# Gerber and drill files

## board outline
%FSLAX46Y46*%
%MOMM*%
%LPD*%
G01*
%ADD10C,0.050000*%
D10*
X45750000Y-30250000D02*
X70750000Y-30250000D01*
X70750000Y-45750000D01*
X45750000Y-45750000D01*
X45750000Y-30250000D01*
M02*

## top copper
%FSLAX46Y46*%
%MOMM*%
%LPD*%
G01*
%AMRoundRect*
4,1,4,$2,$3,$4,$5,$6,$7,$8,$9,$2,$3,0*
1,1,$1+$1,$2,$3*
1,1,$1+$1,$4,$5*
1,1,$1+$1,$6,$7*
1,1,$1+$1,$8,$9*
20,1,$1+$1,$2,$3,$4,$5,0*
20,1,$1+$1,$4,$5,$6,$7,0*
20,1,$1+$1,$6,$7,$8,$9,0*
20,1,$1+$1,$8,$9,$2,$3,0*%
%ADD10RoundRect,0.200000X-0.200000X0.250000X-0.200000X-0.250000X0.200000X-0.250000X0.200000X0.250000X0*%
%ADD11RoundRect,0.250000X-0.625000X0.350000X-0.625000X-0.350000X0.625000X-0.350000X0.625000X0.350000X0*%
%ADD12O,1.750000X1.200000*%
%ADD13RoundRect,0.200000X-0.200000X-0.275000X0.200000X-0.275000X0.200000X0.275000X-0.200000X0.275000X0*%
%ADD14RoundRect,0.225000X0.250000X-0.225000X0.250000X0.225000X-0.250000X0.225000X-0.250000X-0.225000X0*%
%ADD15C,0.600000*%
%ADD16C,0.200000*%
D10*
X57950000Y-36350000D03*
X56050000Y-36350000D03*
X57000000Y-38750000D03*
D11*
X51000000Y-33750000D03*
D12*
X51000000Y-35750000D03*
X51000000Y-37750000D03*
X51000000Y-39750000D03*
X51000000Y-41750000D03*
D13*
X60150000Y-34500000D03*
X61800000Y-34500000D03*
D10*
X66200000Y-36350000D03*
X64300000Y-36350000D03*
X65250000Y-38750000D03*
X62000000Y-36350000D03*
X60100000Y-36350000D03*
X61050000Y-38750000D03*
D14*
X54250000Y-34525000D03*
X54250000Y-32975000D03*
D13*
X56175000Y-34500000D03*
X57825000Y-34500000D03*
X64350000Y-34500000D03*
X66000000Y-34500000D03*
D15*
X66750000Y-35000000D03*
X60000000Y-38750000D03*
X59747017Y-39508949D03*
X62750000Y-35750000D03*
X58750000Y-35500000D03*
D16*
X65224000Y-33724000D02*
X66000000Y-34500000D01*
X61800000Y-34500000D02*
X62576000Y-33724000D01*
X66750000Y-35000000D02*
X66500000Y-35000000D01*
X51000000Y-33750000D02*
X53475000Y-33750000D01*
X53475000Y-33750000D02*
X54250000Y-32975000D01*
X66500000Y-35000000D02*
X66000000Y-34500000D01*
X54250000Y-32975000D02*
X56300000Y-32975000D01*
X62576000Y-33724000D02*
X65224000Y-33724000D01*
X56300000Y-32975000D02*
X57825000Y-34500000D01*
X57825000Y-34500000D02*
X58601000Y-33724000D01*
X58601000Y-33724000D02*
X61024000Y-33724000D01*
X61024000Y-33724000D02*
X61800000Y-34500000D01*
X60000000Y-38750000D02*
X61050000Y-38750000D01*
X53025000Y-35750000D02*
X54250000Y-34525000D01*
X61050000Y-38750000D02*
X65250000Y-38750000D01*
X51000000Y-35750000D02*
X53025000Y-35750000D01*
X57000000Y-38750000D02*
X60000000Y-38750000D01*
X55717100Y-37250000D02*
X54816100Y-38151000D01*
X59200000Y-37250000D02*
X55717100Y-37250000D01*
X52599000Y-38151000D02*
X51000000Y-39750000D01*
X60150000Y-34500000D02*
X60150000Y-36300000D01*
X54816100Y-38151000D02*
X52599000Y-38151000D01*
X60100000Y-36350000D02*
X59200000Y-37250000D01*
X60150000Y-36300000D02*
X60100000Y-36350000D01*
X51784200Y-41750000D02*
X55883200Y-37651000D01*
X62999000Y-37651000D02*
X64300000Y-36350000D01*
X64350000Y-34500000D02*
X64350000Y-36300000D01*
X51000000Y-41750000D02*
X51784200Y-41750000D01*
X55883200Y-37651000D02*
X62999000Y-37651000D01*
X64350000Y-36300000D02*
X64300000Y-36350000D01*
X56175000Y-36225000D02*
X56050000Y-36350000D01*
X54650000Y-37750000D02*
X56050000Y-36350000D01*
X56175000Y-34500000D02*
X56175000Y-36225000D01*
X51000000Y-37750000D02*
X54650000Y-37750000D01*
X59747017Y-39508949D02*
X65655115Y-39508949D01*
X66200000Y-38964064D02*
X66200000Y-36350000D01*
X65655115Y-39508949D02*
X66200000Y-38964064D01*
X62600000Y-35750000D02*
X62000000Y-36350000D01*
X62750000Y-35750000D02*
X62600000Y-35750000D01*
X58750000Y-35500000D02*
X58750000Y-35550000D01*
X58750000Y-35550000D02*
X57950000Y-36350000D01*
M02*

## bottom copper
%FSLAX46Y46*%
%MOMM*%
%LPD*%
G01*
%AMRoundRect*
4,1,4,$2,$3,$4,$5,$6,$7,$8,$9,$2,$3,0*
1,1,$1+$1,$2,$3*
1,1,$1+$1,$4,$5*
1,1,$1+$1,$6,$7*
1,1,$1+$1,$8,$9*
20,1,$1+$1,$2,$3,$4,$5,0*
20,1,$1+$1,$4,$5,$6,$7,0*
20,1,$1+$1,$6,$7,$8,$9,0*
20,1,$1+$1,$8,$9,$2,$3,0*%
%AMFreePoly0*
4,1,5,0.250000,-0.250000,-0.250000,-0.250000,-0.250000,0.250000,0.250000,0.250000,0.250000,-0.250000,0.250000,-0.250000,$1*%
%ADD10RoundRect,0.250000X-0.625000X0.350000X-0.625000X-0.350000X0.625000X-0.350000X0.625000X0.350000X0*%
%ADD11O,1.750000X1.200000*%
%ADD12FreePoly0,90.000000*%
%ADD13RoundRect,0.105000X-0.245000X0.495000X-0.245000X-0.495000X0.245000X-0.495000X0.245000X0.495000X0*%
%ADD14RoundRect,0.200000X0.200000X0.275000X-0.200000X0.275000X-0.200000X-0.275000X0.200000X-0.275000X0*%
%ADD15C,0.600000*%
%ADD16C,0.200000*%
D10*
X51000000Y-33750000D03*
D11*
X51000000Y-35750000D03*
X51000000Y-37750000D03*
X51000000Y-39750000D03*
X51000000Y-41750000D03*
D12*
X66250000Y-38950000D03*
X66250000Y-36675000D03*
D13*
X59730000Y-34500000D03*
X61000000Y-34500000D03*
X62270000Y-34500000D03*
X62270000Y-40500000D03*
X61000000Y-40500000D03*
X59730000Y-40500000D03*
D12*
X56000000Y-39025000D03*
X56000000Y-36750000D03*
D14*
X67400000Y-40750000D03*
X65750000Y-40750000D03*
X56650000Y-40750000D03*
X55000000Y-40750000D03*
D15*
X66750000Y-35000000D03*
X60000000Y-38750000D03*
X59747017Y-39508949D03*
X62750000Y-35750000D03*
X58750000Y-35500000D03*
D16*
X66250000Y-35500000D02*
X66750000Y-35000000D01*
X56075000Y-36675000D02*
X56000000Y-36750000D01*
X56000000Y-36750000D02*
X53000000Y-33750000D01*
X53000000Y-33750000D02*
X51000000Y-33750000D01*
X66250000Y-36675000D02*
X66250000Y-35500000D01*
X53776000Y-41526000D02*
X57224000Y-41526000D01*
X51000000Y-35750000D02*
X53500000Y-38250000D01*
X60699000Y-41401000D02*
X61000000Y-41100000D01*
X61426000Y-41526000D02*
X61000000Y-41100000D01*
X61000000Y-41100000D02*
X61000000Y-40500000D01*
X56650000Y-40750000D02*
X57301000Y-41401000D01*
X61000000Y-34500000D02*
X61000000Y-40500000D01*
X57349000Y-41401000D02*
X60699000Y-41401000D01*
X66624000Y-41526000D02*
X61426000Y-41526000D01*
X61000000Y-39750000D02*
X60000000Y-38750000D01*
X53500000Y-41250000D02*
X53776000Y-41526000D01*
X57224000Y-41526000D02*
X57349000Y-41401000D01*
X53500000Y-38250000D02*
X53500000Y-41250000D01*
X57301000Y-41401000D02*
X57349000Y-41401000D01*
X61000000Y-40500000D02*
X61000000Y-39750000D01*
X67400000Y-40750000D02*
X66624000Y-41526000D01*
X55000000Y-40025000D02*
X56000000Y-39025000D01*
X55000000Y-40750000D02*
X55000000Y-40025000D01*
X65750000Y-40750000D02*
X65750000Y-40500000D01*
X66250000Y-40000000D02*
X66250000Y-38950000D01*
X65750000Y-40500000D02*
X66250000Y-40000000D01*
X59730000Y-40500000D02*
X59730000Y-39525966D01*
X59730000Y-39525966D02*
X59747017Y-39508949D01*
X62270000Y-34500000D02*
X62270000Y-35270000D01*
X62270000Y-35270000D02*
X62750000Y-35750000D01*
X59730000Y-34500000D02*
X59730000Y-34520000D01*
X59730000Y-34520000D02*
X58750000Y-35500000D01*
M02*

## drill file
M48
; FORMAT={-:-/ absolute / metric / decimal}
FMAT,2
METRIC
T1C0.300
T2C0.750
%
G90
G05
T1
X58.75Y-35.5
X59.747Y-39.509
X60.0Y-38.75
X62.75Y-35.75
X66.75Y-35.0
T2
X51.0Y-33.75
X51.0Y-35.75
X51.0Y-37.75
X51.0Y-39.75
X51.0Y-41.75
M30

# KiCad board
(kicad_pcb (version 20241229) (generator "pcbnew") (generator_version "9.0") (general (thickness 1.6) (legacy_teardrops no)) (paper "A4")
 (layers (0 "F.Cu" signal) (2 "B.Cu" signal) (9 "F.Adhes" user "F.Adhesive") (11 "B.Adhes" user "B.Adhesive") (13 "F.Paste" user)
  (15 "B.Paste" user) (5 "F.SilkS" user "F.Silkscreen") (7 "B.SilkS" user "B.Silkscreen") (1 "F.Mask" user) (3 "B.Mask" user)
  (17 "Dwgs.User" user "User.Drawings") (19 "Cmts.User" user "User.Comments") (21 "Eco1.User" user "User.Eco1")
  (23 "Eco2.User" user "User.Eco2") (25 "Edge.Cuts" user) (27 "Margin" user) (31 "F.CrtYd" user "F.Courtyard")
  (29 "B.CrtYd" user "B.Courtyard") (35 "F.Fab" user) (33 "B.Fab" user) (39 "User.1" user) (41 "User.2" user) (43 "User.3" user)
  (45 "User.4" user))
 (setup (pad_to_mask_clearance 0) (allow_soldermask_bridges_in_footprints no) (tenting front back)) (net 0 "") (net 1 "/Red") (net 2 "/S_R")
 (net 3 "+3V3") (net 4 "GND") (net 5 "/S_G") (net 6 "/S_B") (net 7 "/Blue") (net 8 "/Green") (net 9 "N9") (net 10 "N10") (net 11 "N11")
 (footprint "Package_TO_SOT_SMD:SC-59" (layer "F.Cu") (at 57 37.55 -90)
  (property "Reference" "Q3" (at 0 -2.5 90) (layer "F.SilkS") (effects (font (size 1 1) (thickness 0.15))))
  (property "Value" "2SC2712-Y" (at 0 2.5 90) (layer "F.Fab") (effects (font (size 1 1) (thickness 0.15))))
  (pad "1" smd roundrect (at -1.2 -0.95 270) (size 0.9 0.8) (layers "F.Cu" "F.Mask" "F.Paste") (roundrect_rratio 0.25) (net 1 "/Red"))
  (pad "2" smd roundrect (at -1.2 0.95 270) (size 0.9 0.8) (layers "F.Cu" "F.Mask" "F.Paste") (roundrect_rratio 0.25) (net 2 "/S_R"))
  (pad "3" smd roundrect (at 1.2 0 270) (size 0.9 0.8) (layers "F.Cu" "F.Mask" "F.Paste") (roundrect_rratio 0.25) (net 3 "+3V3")))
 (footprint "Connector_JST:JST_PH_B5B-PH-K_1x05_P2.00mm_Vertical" (layer "F.Cu") (at 51 33.75 -90)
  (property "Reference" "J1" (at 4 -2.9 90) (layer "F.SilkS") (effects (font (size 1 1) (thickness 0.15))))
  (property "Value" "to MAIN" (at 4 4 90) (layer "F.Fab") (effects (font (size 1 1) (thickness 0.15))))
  (pad "1" thru_hole roundrect (at 0 0 270) (size 1.2 1.75) (drill 0.75) (layers "*.Cu" "*.Mask") (remove_unused_layers no)
   (roundrect_rratio 0.208333) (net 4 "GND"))
  (pad "2" thru_hole oval (at 2 0 270) (size 1.2 1.75) (drill 0.75) (layers "*.Cu" "*.Mask") (remove_unused_layers no) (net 3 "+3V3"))
  (pad "3" thru_hole oval (at 4 0 270) (size 1.2 1.75) (drill 0.75) (layers "*.Cu" "*.Mask") (remove_unused_layers no) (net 2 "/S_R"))
  (pad "4" thru_hole oval (at 6 0 270) (size 1.2 1.75) (drill 0.75) (layers "*.Cu" "*.Mask") (remove_unused_layers no) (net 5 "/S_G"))
  (pad "5" thru_hole oval (at 8 0 270) (size 1.2 1.75) (drill 0.75) (layers "*.Cu" "*.Mask") (remove_unused_layers no) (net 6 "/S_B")))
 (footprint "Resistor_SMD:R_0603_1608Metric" (layer "F.Cu") (at 60.975 34.5)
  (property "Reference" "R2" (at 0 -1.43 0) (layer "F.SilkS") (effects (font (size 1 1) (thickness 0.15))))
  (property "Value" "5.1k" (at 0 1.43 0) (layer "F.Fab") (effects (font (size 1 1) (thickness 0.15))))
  (pad "1" smd roundrect (at -0.825 0) (size 0.8 0.95) (layers "F.Cu" "F.Mask" "F.Paste") (roundrect_rratio 0.25) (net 5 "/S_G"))
  (pad "2" smd roundrect (at 0.825 0) (size 0.8 0.95) (layers "F.Cu" "F.Mask" "F.Paste") (roundrect_rratio 0.25) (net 4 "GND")))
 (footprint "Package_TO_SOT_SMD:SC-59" (layer "F.Cu") (at 65.25 37.55 -90)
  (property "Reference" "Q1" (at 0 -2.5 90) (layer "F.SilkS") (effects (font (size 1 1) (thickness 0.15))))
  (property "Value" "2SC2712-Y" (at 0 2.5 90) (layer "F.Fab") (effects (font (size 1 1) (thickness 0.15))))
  (pad "1" smd roundrect (at -1.2 -0.95 270) (size 0.9 0.8) (layers "F.Cu" "F.Mask" "F.Paste") (roundrect_rratio 0.25) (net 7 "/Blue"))
  (pad "2" smd roundrect (at -1.2 0.95 270) (size 0.9 0.8) (layers "F.Cu" "F.Mask" "F.Paste") (roundrect_rratio 0.25) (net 6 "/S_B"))
  (pad "3" smd roundrect (at 1.2 0 270) (size 0.9 0.8) (layers "F.Cu" "F.Mask" "F.Paste") (roundrect_rratio 0.25) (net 3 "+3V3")))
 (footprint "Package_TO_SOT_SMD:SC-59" (layer "F.Cu") (at 61.05 37.55 -90)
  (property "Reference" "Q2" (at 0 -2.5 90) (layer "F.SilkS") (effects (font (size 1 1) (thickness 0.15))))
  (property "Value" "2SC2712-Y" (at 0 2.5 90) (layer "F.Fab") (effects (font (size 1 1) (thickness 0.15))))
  (pad "1" smd roundrect (at -1.2 -0.95 270) (size 0.9 0.8) (layers "F.Cu" "F.Mask" "F.Paste") (roundrect_rratio 0.25) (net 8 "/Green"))
  (pad "2" smd roundrect (at -1.2 0.95 270) (size 0.9 0.8) (layers "F.Cu" "F.Mask" "F.Paste") (roundrect_rratio 0.25) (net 5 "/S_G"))
  (pad "3" smd roundrect (at 1.2 0 270) (size 0.9 0.8) (layers "F.Cu" "F.Mask" "F.Paste") (roundrect_rratio 0.25) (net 3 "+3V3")))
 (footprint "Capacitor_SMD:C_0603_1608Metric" (layer "F.Cu") (at 54.25 33.75 90)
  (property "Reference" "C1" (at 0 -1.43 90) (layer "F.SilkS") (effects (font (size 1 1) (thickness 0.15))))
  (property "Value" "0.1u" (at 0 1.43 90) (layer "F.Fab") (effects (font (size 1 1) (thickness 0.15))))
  (pad "1" smd roundrect (at -0.775 0 90) (size 0.9 0.95) (layers "F.Cu" "F.Mask" "F.Paste") (roundrect_rratio 0.25) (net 3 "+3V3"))
  (pad "2" smd roundrect (at 0.775 0 90) (size 0.9 0.95) (layers "F.Cu" "F.Mask" "F.Paste") (roundrect_rratio 0.25) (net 4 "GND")))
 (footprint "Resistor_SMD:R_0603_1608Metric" (layer "F.Cu") (at 57 34.5)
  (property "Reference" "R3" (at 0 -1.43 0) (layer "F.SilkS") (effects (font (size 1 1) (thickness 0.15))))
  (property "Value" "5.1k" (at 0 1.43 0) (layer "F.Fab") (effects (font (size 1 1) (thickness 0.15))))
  (pad "1" smd roundrect (at -0.825 0) (size 0.8 0.95) (layers "F.Cu" "F.Mask" "F.Paste") (roundrect_rratio 0.25) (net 2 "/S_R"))
  (pad "2" smd roundrect (at 0.825 0) (size 0.8 0.95) (layers "F.Cu" "F.Mask" "F.Paste") (roundrect_rratio 0.25) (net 4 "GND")))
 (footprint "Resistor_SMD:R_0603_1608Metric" (layer "F.Cu") (at 65.175 34.5)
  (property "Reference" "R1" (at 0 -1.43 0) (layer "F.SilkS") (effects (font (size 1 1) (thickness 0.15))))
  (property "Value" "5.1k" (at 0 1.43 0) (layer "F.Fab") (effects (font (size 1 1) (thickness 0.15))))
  (pad "1" smd roundrect (at -0.825 0) (size 0.8 0.95) (layers "F.Cu" "F.Mask" "F.Paste") (roundrect_rratio 0.25) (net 6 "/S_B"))
  (pad "2" smd roundrect (at 0.825 0) (size 0.8 0.95) (layers "F.Cu" "F.Mask" "F.Paste") (roundrect_rratio 0.25) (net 4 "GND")))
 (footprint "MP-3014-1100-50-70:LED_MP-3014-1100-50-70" (layer "B.Cu") (at 66.25 37.5 90)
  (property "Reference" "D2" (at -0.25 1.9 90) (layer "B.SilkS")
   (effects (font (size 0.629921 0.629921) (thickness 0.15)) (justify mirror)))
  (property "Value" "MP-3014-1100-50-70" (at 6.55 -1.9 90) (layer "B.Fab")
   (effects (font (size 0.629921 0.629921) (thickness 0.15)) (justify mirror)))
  (pad "A" smd custom (at -1.45 0 90) (size 0.5 0.5) (layers "B.Cu") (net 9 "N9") (options (clearance outline) (anchor rect)) (primitives))
  (pad "C" smd custom (at 0.825 0 90) (size 0.5 0.5) (layers "B.Cu") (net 4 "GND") (options (clearance outline) (anchor rect)) (primitives)))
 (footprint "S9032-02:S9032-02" (layer "B.Cu") (at 61 37.5 -90)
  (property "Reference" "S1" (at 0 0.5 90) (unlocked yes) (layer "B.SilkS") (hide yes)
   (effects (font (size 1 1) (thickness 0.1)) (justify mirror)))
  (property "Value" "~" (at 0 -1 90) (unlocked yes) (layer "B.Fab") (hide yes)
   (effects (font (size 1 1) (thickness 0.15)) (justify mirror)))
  (pad "1" smd roundrect (at -3 1.27 270) (size 1.2 0.7) (layers "B.Cu" "B.Mask" "B.Paste") (roundrect_rratio 0.15) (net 1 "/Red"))
  (pad "2" smd roundrect (at -3 0 270) (size 1.2 0.7) (layers "B.Cu" "B.Mask" "B.Paste") (roundrect_rratio 0.15) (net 3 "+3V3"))
  (pad "3" smd roundrect (at -3 -1.27 270) (size 1.2 0.7) (layers "B.Cu" "B.Mask" "B.Paste") (roundrect_rratio 0.15) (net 8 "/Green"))
  (pad "4" smd roundrect (at 3 -1.27 270) (size 1.2 0.7) (layers "B.Cu" "B.Mask" "B.Paste") (roundrect_rratio 0.15) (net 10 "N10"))
  (pad "5" smd roundrect (at 3 0 270) (size 1.2 0.7) (layers "B.Cu" "B.Mask" "B.Paste") (roundrect_rratio 0.15) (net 3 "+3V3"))
  (pad "6" smd roundrect (at 3 1.27 270) (size 1.2 0.7) (layers "B.Cu" "B.Mask" "B.Paste") (roundrect_rratio 0.15) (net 7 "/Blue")))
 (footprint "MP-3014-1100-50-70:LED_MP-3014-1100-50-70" (layer "B.Cu") (at 56 37.575 90)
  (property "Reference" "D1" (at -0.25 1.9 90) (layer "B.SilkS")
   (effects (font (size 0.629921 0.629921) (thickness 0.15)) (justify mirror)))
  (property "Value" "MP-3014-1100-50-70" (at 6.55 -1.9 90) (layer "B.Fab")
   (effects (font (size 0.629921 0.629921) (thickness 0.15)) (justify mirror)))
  (pad "A" smd custom (at -1.45 0 90) (size 0.5 0.5) (layers "B.Cu") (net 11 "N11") (options (clearance outline) (anchor rect)) (primitives))
  (pad "C" smd custom (at 0.825 0 90) (size 0.5 0.5) (layers "B.Cu") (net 4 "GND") (options (clearance outline) (anchor rect)) (primitives)))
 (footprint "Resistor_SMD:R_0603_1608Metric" (layer "B.Cu") (at 66.575 40.75 180)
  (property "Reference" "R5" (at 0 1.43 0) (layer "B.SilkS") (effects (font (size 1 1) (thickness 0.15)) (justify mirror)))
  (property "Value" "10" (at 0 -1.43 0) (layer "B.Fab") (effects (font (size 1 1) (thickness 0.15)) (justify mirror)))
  (pad "1" smd roundrect (at -0.825 0 180) (size 0.8 0.95) (layers "B.Cu" "B.Mask" "B.Paste") (roundrect_rratio 0.25) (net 3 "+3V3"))
  (pad "2" smd roundrect (at 0.825 0 180) (size 0.8 0.95) (layers "B.Cu" "B.Mask" "B.Paste") (roundrect_rratio 0.25) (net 9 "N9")))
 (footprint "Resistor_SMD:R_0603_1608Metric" (layer "B.Cu") (at 55.825 40.75 180)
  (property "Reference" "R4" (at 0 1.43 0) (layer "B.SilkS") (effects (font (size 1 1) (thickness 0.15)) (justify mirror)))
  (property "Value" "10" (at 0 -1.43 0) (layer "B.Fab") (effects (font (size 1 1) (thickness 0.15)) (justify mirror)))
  (pad "1" smd roundrect (at -0.825 0 180) (size 0.8 0.95) (layers "B.Cu" "B.Mask" "B.Paste") (roundrect_rratio 0.25) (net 3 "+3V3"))
  (pad "2" smd roundrect (at 0.825 0 180) (size 0.8 0.95) (layers "B.Cu" "B.Mask" "B.Paste") (roundrect_rratio 0.25) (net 11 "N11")))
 (gr_rect (start 45.75 30.25) (end 70.75 45.75) (stroke (width 0.05) (type default)) (fill no) (layer "Edge.Cuts"))
 (segment (start 65.224 33.724) (end 66 34.5) (width 0.2) (layer "F.Cu") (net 4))
 (segment (start 61.8 34.5) (end 62.576 33.724) (width 0.2) (layer "F.Cu") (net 4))
 (segment (start 66.75 35) (end 66.5 35) (width 0.2) (layer "F.Cu") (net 4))
 (segment (start 51 33.75) (end 53.475 33.75) (width 0.2) (layer "F.Cu") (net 4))
 (segment (start 53.475 33.75) (end 54.25 32.975) (width 0.2) (layer "F.Cu") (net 4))
 (segment (start 66.5 35) (end 66 34.5) (width 0.2) (layer "F.Cu") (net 4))
 (segment (start 54.25 32.975) (end 56.3 32.975) (width 0.2) (layer "F.Cu") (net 4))
 (segment (start 62.576 33.724) (end 65.224 33.724) (width 0.2) (layer "F.Cu") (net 4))
 (segment (start 56.3 32.975) (end 57.825 34.5) (width 0.2) (layer "F.Cu") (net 4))
 (segment (start 57.825 34.5) (end 58.601 33.724) (width 0.2) (layer "F.Cu") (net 4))
 (segment (start 58.601 33.724) (end 61.024 33.724) (width 0.2) (layer "F.Cu") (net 4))
 (segment (start 61.024 33.724) (end 61.8 34.5) (width 0.2) (layer "F.Cu") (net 4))
 (via (at 66.75 35) (size 0.6) (drill 0.3) (layers "F.Cu" "B.Cu") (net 4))
 (segment (start 66.25 35.5) (end 66.75 35) (width 0.2) (layer "B.Cu") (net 4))
 (segment (start 56.075 36.675) (end 56 36.75) (width 0.2) (layer "B.Cu") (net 4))
 (segment (start 56 36.75) (end 53 33.75) (width 0.2) (layer "B.Cu") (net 4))
 (segment (start 53 33.75) (end 51 33.75) (width 0.2) (layer "B.Cu") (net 4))
 (segment (start 66.25 36.675) (end 66.25 35.5) (width 0.2) (layer "B.Cu") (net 4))
 (segment (start 60 38.75) (end 61.05 38.75) (width 0.2) (layer "F.Cu") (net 3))
 (segment (start 53.025 35.75) (end 54.25 34.525) (width 0.2) (layer "F.Cu") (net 3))
 (segment (start 61.05 38.75) (end 65.25 38.75) (width 0.2) (layer "F.Cu") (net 3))
 (segment (start 51 35.75) (end 53.025 35.75) (width 0.2) (layer "F.Cu") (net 3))
 (segment (start 57 38.75) (end 60 38.75) (width 0.2) (layer "F.Cu") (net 3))
 (via (at 60 38.75) (size 0.6) (drill 0.3) (layers "F.Cu" "B.Cu") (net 3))
 (segment (start 53.776 41.526) (end 57.224 41.526) (width 0.2) (layer "B.Cu") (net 3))
 (segment (start 51 35.75) (end 53.5 38.25) (width 0.2) (layer "B.Cu") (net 3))
 (segment (start 60.699 41.401) (end 61 41.1) (width 0.2) (layer "B.Cu") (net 3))
 (segment (start 61.426 41.526) (end 61 41.1) (width 0.2) (layer "B.Cu") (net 3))
 (segment (start 61 41.1) (end 61 40.5) (width 0.2) (layer "B.Cu") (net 3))
 (segment (start 56.65 40.75) (end 57.301 41.401) (width 0.2) (layer "B.Cu") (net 3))
 (segment (start 61 34.5) (end 61 40.5) (width 0.2) (layer "B.Cu") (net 3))
 (segment (start 57.349 41.401) (end 60.699 41.401) (width 0.2) (layer "B.Cu") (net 3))
 (segment (start 66.624 41.526) (end 61.426 41.526) (width 0.2) (layer "B.Cu") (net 3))
 (segment (start 61 39.75) (end 60 38.75) (width 0.2) (layer "B.Cu") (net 3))
 (segment (start 53.5 41.25) (end 53.776 41.526) (width 0.2) (layer "B.Cu") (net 3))
 (segment (start 57.224 41.526) (end 57.349 41.401) (width 0.2) (layer "B.Cu") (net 3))
 (segment (start 53.5 38.25) (end 53.5 41.25) (width 0.2) (layer "B.Cu") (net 3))
 (segment (start 57.301 41.401) (end 57.349 41.401) (width 0.2) (layer "B.Cu") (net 3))
 (segment (start 61 40.5) (end 61 39.75) (width 0.2) (layer "B.Cu") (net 3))
 (segment (start 67.4 40.75) (end 66.624 41.526) (width 0.2) (layer "B.Cu") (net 3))
 (segment (start 55 40.025) (end 56 39.025) (width 0.2) (layer "B.Cu") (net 11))
 (segment (start 55 40.75) (end 55 40.025) (width 0.2) (layer "B.Cu") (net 11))
 (segment (start 65.75 40.75) (end 65.75 40.5) (width 0.2) (layer "B.Cu") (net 9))
 (segment (start 66.25 40) (end 66.25 38.95) (width 0.2) (layer "B.Cu") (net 9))
 (segment (start 65.75 40.5) (end 66.25 40) (width 0.2) (layer "B.Cu") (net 9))
 (segment (start 55.7171 37.25) (end 54.8161 38.151) (width 0.2) (layer "F.Cu") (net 5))
 (segment (start 59.2 37.25) (end 55.7171 37.25) (width 0.2) (layer "F.Cu") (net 5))
 (segment (start 52.599 38.151) (end 51 39.75) (width 0.2) (layer "F.Cu") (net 5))
 (segment (start 60.15 34.5) (end 60.15 36.3) (width 0.2) (layer "F.Cu") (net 5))
 (segment (start 54.8161 38.151) (end 52.599 38.151) (width 0.2) (layer "F.Cu") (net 5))
 (segment (start 60.1 36.35) (end 59.2 37.25) (width 0.2) (layer "F.Cu") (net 5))
 (segment (start 60.15 36.3) (end 60.1 36.35) (width 0.2) (layer "F.Cu") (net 5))
 (segment (start 51.7842 41.75) (end 55.8832 37.651) (width 0.2) (layer "F.Cu") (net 6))
 (segment (start 62.999 37.651) (end 64.3 36.35) (width 0.2) (layer "F.Cu") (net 6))
 (segment (start 64.35 34.5) (end 64.35 36.3) (width 0.2) (layer "F.Cu") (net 6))
 (segment (start 51 41.75) (end 51.7842 41.75) (width 0.2) (layer "F.Cu") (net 6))
 (segment (start 55.8832 37.651) (end 62.999 37.651) (width 0.2) (layer "F.Cu") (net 6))
 (segment (start 64.35 36.3) (end 64.3 36.35) (width 0.2) (layer "F.Cu") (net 6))
 (segment (start 56.175 36.225) (end 56.05 36.35) (width 0.2) (layer "F.Cu") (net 2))
 (segment (start 54.65 37.75) (end 56.05 36.35) (width 0.2) (layer "F.Cu") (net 2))
 (segment (start 56.175 34.5) (end 56.175 36.225) (width 0.2) (layer "F.Cu") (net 2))
 (segment (start 51 37.75) (end 54.65 37.75) (width 0.2) (layer "F.Cu") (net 2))
 (segment (start 59.747017 39.508949) (end 65.655115 39.508949) (width 0.2) (layer "F.Cu") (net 7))
 (segment (start 66.2 38.964064) (end 66.2 36.35) (width 0.2) (layer "F.Cu") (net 7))
 (segment (start 65.655115 39.508949) (end 66.2 38.964064) (width 0.2) (layer "F.Cu") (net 7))
 (via (at 59.747017 39.508949) (size 0.6) (drill 0.3) (layers "F.Cu" "B.Cu") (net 7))
 (segment (start 59.73 40.5) (end 59.73 39.525966) (width 0.2) (layer "B.Cu") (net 7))
 (segment (start 59.73 39.525966) (end 59.747017 39.508949) (width 0.2) (layer "B.Cu") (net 7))
 (segment (start 62.6 35.75) (end 62 36.35) (width 0.2) (layer "F.Cu") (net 8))
 (segment (start 62.75 35.75) (end 62.6 35.75) (width 0.2) (layer "F.Cu") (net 8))
 (via (at 62.75 35.75) (size 0.6) (drill 0.3) (layers "F.Cu" "B.Cu") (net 8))
 (segment (start 62.27 34.5) (end 62.27 35.27) (width 0.2) (layer "B.Cu") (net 8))
 (segment (start 62.27 35.27) (end 62.75 35.75) (width 0.2) (layer "B.Cu") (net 8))
 (segment (start 58.75 35.5) (end 58.75 35.55) (width 0.2) (layer "F.Cu") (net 1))
 (segment (start 58.75 35.55) (end 57.95 36.35) (width 0.2) (layer "F.Cu") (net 1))
 (via (at 58.75 35.5) (size 0.6) (drill 0.3) (layers "F.Cu" "B.Cu") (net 1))
 (segment (start 59.73 34.5) (end 59.73 34.52) (width 0.2) (layer "B.Cu") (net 1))
 (segment (start 59.73 34.52) (end 58.75 35.5) (width 0.2) (layer "B.Cu") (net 1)))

